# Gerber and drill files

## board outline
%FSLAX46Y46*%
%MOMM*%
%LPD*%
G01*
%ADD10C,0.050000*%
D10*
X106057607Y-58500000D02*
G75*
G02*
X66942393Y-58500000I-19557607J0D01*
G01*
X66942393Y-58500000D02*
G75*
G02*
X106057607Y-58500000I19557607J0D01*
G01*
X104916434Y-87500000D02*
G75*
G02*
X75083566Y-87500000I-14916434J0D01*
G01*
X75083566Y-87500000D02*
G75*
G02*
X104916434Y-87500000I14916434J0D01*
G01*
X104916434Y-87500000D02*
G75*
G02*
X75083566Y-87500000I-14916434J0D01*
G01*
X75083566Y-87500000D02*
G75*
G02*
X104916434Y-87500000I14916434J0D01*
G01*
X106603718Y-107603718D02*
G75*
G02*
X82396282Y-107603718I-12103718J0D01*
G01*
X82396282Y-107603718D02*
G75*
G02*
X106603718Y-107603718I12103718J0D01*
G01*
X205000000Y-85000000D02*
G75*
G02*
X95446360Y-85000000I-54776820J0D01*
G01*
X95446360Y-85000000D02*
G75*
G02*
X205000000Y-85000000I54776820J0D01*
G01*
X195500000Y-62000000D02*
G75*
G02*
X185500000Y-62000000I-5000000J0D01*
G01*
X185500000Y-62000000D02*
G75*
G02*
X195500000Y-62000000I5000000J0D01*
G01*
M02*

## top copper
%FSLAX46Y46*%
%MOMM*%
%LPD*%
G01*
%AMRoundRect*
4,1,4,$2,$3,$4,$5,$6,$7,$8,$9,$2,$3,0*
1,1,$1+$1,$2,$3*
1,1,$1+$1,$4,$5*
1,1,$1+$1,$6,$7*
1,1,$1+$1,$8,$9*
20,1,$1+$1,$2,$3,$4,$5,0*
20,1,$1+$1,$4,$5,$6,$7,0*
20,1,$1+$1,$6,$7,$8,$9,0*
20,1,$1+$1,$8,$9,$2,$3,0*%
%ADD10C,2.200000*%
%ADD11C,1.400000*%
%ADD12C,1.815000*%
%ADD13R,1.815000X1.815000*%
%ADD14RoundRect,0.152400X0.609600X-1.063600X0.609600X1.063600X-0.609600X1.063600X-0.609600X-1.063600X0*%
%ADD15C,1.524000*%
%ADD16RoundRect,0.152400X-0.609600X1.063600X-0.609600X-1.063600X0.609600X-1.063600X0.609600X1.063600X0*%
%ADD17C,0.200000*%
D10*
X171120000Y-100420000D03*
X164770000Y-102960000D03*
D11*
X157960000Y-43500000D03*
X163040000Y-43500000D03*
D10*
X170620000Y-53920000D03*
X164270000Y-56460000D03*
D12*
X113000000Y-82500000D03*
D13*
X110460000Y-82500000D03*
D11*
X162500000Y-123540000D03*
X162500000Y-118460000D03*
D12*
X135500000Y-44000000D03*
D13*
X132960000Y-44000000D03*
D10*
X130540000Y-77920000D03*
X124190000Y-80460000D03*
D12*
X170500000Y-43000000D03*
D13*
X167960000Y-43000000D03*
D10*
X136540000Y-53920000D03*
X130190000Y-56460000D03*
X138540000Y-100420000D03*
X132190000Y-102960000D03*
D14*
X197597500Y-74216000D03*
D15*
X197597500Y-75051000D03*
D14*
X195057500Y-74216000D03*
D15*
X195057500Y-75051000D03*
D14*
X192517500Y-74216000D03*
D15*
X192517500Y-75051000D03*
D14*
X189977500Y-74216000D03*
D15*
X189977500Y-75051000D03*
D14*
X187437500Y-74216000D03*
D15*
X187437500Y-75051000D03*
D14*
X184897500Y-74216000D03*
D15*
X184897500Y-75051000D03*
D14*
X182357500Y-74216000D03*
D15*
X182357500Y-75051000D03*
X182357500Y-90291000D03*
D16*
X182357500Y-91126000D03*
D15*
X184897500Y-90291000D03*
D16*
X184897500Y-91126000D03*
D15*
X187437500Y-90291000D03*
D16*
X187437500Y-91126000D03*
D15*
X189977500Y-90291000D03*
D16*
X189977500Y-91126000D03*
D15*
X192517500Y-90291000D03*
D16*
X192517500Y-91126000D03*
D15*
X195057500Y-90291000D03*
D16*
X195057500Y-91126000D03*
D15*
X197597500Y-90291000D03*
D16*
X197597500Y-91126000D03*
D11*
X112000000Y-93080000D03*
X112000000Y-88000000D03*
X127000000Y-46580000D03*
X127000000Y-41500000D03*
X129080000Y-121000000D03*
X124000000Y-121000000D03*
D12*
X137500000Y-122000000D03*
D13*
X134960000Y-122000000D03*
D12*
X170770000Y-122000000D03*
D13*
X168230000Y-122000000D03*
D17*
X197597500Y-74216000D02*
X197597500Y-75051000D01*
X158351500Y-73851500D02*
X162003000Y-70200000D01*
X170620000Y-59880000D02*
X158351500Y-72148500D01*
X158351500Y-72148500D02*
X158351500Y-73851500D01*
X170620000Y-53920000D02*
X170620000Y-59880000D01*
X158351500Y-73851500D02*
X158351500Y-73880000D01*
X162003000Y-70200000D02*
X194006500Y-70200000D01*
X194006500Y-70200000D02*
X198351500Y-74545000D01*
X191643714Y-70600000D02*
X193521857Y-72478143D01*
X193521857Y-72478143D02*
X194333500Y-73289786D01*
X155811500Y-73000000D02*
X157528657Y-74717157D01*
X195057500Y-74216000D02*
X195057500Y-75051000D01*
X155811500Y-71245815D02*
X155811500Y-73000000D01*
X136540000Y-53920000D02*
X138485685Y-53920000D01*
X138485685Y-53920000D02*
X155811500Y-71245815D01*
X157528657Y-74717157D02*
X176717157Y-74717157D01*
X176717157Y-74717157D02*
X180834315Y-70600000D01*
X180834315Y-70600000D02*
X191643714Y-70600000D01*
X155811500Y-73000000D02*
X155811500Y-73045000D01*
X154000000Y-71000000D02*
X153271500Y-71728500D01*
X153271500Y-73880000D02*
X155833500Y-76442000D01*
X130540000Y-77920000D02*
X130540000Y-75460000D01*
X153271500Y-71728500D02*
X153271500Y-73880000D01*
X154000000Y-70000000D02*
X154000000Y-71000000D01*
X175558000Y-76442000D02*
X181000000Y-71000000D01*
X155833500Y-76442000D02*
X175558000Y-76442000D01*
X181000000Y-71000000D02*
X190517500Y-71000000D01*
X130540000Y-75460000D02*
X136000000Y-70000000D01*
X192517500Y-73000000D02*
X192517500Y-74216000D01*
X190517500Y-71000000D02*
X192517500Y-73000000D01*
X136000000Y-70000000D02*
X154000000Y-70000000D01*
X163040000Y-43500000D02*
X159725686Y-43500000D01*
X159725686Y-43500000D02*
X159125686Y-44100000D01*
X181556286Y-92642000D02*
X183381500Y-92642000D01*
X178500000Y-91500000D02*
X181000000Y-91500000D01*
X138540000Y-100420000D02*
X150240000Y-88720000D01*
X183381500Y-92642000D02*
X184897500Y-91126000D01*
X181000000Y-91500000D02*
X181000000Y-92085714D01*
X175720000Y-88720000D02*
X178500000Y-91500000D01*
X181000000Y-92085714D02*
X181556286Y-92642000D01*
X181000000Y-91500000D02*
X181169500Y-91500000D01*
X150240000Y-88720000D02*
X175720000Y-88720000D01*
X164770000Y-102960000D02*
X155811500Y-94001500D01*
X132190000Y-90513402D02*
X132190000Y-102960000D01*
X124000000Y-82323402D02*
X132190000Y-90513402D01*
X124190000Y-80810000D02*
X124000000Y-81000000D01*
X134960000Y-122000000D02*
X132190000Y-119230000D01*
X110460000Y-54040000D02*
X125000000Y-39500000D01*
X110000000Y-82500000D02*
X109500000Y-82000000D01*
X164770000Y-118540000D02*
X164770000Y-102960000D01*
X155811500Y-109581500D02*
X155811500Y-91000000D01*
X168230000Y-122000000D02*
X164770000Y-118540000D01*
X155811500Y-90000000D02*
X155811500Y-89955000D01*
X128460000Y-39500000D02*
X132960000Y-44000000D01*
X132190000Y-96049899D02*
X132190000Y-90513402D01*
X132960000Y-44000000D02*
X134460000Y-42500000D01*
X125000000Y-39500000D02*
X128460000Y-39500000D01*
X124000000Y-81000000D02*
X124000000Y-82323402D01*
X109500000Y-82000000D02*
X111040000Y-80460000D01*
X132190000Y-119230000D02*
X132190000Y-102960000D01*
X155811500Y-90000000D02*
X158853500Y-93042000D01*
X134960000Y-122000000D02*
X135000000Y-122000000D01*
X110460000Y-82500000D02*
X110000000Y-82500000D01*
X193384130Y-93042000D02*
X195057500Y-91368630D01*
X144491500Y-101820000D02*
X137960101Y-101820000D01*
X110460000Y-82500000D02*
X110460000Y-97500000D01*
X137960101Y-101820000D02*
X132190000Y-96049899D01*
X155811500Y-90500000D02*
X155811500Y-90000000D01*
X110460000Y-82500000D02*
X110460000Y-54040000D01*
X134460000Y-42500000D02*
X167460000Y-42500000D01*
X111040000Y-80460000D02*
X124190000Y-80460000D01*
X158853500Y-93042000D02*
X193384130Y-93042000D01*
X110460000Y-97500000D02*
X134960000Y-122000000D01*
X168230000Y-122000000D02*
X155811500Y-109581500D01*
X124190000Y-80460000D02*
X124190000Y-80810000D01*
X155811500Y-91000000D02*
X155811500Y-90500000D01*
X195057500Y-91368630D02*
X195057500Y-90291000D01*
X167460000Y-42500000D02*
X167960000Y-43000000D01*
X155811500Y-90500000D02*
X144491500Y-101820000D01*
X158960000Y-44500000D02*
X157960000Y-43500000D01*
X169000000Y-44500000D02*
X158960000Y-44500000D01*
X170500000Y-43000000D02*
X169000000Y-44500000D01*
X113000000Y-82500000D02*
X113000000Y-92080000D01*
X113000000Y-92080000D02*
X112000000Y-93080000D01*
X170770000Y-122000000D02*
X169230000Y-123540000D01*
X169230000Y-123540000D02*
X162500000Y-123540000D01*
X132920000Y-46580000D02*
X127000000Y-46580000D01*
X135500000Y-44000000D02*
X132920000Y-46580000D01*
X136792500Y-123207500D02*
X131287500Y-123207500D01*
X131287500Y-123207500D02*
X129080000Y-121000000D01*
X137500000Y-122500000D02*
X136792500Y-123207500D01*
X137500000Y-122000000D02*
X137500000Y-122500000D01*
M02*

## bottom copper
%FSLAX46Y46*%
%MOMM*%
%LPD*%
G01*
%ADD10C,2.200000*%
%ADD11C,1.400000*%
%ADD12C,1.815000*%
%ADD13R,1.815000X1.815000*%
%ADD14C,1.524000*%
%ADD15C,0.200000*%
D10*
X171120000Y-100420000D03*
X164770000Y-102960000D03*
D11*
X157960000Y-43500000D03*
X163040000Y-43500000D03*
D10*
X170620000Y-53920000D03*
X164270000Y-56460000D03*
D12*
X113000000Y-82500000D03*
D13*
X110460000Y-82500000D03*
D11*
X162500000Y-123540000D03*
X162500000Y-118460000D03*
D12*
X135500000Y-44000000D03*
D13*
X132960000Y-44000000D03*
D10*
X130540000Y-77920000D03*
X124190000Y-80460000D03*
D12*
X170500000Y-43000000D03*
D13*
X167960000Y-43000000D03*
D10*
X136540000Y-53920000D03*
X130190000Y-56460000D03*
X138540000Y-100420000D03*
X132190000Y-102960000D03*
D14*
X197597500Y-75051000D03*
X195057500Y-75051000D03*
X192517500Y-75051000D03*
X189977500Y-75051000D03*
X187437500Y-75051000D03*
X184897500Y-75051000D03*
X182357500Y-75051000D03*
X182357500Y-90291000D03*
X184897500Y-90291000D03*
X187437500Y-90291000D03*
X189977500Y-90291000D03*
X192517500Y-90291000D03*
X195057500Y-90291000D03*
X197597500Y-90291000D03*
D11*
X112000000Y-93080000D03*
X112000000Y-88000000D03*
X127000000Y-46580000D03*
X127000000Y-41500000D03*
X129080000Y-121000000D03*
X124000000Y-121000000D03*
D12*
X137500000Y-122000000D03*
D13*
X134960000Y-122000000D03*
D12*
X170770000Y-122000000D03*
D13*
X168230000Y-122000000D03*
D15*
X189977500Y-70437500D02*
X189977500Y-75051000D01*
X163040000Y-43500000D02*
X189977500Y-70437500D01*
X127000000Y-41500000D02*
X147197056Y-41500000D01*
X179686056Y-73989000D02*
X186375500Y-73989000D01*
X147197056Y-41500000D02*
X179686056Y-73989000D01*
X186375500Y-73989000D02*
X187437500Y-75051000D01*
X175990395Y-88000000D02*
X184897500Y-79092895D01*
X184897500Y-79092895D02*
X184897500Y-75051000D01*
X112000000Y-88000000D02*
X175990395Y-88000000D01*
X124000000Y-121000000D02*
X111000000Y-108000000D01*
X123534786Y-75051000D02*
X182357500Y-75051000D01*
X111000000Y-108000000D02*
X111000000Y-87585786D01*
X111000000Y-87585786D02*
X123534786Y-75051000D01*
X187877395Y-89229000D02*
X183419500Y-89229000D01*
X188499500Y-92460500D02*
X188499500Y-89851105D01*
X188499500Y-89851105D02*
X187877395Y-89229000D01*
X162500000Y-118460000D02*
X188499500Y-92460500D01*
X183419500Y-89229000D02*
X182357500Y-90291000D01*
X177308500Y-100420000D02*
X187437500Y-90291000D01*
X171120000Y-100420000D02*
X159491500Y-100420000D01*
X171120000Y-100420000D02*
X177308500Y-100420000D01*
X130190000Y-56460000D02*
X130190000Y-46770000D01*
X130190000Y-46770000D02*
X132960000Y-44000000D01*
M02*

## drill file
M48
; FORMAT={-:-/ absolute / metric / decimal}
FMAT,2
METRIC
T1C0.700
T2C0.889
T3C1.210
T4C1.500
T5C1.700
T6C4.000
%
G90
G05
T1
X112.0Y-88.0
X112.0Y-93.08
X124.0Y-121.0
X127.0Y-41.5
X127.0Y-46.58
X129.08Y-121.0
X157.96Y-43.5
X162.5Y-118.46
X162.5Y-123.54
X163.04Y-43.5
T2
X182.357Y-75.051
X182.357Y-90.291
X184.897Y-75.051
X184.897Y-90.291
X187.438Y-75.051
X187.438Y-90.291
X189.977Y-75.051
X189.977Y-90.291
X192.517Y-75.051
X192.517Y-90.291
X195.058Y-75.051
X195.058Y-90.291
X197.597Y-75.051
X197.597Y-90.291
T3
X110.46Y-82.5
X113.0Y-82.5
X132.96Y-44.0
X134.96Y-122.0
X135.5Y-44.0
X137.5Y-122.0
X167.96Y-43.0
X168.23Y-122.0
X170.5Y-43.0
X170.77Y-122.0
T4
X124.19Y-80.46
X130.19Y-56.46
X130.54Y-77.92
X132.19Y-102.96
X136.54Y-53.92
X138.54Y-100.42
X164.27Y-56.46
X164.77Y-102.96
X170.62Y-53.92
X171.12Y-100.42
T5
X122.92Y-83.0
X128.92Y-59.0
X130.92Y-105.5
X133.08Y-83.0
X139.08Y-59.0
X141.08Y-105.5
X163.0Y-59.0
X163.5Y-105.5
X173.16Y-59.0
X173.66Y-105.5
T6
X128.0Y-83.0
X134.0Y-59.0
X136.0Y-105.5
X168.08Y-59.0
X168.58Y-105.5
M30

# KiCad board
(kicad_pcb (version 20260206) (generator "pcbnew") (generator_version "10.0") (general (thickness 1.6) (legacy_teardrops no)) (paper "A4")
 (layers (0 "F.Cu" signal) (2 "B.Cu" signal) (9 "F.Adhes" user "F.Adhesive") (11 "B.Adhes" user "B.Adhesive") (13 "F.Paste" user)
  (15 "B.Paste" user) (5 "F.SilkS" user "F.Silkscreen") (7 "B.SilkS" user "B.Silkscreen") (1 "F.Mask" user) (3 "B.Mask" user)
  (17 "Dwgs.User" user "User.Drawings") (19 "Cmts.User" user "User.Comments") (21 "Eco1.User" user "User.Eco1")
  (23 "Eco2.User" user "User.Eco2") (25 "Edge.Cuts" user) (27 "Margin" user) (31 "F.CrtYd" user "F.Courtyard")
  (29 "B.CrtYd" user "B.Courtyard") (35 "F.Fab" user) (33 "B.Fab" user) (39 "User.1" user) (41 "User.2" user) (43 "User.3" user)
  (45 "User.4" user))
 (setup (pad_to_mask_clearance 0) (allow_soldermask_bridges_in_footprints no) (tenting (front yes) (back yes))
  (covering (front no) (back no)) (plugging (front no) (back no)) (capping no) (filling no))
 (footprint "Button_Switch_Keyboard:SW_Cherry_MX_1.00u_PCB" (layer "F.Cu") (at 171.12 100.42)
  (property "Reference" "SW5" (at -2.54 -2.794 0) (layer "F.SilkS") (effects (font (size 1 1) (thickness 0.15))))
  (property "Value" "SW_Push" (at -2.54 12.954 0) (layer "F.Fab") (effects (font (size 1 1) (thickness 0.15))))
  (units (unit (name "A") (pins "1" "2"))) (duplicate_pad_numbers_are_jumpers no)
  (pad "" np_thru_hole circle (at -7.62 5.08) (size 1.7 1.7) (drill 1.7) (layers "*.Cu" "*.Mask"))
  (pad "" np_thru_hole circle (at -2.54 5.08) (size 4 4) (drill 4) (layers "*.Cu" "*.Mask"))
  (pad "" np_thru_hole circle (at 2.54 5.08) (size 1.7 1.7) (drill 1.7) (layers "*.Cu" "*.Mask"))
  (pad "1" thru_hole circle (at 0 0) (size 2.2 2.2) (drill 1.5) (layers "*.Cu" "*.Mask") (remove_unused_layers no) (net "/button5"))
  (pad "2" thru_hole circle (at -6.35 2.54) (size 2.2 2.2) (drill 1.5) (layers "*.Cu" "*.Mask") (remove_unused_layers no) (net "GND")))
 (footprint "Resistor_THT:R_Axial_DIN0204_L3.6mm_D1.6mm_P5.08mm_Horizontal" (layer "F.Cu") (at 157.96 43.5)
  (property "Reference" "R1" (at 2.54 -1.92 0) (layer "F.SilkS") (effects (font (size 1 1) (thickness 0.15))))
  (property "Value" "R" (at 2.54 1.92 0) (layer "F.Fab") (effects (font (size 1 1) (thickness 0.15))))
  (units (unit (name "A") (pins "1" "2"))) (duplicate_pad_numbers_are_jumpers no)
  (pad "1" thru_hole circle (at 0 0) (size 1.4 1.4) (drill 0.7) (layers "*.Cu" "*.Mask") (remove_unused_layers no) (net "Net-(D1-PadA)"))
  (pad "2" thru_hole circle (at 5.08 0) (size 1.4 1.4) (drill 0.7) (layers "*.Cu" "*.Mask") (remove_unused_layers no) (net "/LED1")))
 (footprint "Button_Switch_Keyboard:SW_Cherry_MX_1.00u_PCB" (layer "F.Cu") (at 170.62 53.92)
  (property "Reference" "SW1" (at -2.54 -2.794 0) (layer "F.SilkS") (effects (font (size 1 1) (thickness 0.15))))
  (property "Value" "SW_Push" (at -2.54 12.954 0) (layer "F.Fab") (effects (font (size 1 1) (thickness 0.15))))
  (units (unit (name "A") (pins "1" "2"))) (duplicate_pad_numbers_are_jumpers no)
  (pad "" np_thru_hole circle (at -7.62 5.08) (size 1.7 1.7) (drill 1.7) (layers "*.Cu" "*.Mask"))
  (pad "" np_thru_hole circle (at -2.54 5.08) (size 4 4) (drill 4) (layers "*.Cu" "*.Mask"))
  (pad "" np_thru_hole circle (at 2.54 5.08) (size 1.7 1.7) (drill 1.7) (layers "*.Cu" "*.Mask"))
  (pad "1" thru_hole circle (at 0 0) (size 2.2 2.2) (drill 1.5) (layers "*.Cu" "*.Mask") (remove_unused_layers no) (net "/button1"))
  (pad "2" thru_hole circle (at -6.35 2.54) (size 2.2 2.2) (drill 1.5) (layers "*.Cu" "*.Mask") (remove_unused_layers no) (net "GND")))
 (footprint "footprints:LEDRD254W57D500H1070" (layer "F.Cu") (at 111.73 82.5)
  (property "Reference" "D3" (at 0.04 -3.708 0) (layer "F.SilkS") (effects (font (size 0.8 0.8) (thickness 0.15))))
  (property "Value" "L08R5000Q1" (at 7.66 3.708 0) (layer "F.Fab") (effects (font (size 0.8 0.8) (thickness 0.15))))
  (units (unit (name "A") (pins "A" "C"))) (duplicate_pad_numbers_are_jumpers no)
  (pad "A" thru_hole circle (at 1.27 0) (size 1.815 1.815) (drill 1.21) (layers "*.Cu" "*.Mask") (remove_unused_layers no)
   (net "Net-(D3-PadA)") (solder_mask_margin 0.102))
  (pad "C" thru_hole rect (at -1.27 0) (size 1.815 1.815) (drill 1.21) (layers "*.Cu" "*.Mask") (remove_unused_layers no) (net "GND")
   (solder_mask_margin 0.102)))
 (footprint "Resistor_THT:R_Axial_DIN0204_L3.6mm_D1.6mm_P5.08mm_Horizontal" (layer "F.Cu") (at 162.5 123.54 90)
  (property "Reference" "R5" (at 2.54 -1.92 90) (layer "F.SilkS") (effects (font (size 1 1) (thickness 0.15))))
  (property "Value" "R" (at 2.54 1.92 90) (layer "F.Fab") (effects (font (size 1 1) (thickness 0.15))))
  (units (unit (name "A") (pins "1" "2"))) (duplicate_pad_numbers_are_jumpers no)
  (pad "1" thru_hole circle (at 0 0 90) (size 1.4 1.4) (drill 0.7) (layers "*.Cu" "*.Mask") (remove_unused_layers no) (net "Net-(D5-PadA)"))
  (pad "2" thru_hole circle (at 5.08 0 90) (size 1.4 1.4) (drill 0.7) (layers "*.Cu" "*.Mask") (remove_unused_layers no) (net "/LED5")))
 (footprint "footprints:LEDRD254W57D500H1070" (layer "F.Cu") (at 134.23 44)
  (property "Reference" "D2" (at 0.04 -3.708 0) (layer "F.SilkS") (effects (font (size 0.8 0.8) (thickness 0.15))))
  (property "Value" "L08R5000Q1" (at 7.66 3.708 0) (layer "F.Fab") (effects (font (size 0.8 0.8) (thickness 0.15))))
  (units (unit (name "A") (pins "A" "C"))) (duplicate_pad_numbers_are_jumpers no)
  (pad "A" thru_hole circle (at 1.27 0) (size 1.815 1.815) (drill 1.21) (layers "*.Cu" "*.Mask") (remove_unused_layers no)
   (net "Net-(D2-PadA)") (solder_mask_margin 0.102))
  (pad "C" thru_hole rect (at -1.27 0) (size 1.815 1.815) (drill 1.21) (layers "*.Cu" "*.Mask") (remove_unused_layers no) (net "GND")
   (solder_mask_margin 0.102)))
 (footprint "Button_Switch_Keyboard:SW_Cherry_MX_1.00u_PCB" (layer "F.Cu") (at 130.54 77.92)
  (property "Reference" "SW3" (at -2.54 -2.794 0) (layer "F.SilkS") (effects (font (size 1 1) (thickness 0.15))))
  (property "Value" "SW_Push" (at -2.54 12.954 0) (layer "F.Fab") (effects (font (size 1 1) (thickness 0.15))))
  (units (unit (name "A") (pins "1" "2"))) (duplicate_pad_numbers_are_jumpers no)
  (pad "" np_thru_hole circle (at -7.62 5.08) (size 1.7 1.7) (drill 1.7) (layers "*.Cu" "*.Mask"))
  (pad "" np_thru_hole circle (at -2.54 5.08) (size 4 4) (drill 4) (layers "*.Cu" "*.Mask"))
  (pad "" np_thru_hole circle (at 2.54 5.08) (size 1.7 1.7) (drill 1.7) (layers "*.Cu" "*.Mask"))
  (pad "1" thru_hole circle (at 0 0) (size 2.2 2.2) (drill 1.5) (layers "*.Cu" "*.Mask") (remove_unused_layers no) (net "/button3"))
  (pad "2" thru_hole circle (at -6.35 2.54) (size 2.2 2.2) (drill 1.5) (layers "*.Cu" "*.Mask") (remove_unused_layers no) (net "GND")))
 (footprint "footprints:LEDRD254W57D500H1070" (layer "F.Cu") (at 169.23 43)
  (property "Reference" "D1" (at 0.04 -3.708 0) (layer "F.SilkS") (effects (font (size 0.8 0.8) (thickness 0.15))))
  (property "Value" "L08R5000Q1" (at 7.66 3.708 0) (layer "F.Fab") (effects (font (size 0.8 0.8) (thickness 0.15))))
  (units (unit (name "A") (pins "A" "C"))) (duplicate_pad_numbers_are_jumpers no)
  (pad "A" thru_hole circle (at 1.27 0) (size 1.815 1.815) (drill 1.21) (layers "*.Cu" "*.Mask") (remove_unused_layers no)
   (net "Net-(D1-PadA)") (solder_mask_margin 0.102))
  (pad "C" thru_hole rect (at -1.27 0) (size 1.815 1.815) (drill 1.21) (layers "*.Cu" "*.Mask") (remove_unused_layers no) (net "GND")
   (solder_mask_margin 0.102)))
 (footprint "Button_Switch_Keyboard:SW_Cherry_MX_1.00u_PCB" (layer "F.Cu") (at 136.54 53.92)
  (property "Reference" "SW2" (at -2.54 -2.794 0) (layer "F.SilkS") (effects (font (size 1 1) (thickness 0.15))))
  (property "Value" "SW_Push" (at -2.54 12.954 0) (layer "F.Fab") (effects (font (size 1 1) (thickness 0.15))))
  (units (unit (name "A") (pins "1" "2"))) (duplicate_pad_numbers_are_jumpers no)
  (pad "" np_thru_hole circle (at -7.62 5.08) (size 1.7 1.7) (drill 1.7) (layers "*.Cu" "*.Mask"))
  (pad "" np_thru_hole circle (at -2.54 5.08) (size 4 4) (drill 4) (layers "*.Cu" "*.Mask"))
  (pad "" np_thru_hole circle (at 2.54 5.08) (size 1.7 1.7) (drill 1.7) (layers "*.Cu" "*.Mask"))
  (pad "1" thru_hole circle (at 0 0) (size 2.2 2.2) (drill 1.5) (layers "*.Cu" "*.Mask") (remove_unused_layers no) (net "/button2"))
  (pad "2" thru_hole circle (at -6.35 2.54) (size 2.2 2.2) (drill 1.5) (layers "*.Cu" "*.Mask") (remove_unused_layers no) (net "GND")))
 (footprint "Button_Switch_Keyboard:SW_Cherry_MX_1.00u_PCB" (layer "F.Cu") (at 138.54 100.42)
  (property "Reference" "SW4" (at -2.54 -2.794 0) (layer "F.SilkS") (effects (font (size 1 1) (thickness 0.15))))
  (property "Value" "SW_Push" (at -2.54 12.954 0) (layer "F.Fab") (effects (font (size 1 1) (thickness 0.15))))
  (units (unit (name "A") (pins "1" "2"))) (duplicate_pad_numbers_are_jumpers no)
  (pad "" np_thru_hole circle (at -7.62 5.08) (size 1.7 1.7) (drill 1.7) (layers "*.Cu" "*.Mask"))
  (pad "" np_thru_hole circle (at -2.54 5.08) (size 4 4) (drill 4) (layers "*.Cu" "*.Mask"))
  (pad "" np_thru_hole circle (at 2.54 5.08) (size 1.7 1.7) (drill 1.7) (layers "*.Cu" "*.Mask"))
  (pad "1" thru_hole circle (at 0 0) (size 2.2 2.2) (drill 1.5) (layers "*.Cu" "*.Mask") (remove_unused_layers no) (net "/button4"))
  (pad "2" thru_hole circle (at -6.35 2.54) (size 2.2 2.2) (drill 1.5) (layers "*.Cu" "*.Mask") (remove_unused_layers no) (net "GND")))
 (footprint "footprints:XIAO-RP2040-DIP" (layer "F.Cu") (at 189.9775 82.671)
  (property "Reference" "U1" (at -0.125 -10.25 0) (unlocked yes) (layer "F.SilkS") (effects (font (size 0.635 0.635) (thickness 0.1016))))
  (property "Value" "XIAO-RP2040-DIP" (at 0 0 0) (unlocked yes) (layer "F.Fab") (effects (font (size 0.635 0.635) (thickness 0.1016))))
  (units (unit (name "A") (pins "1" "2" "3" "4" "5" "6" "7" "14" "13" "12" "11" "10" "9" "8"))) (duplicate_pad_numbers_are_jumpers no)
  (pad "1" smd roundrect (at 7.62 -8.455 90) (size 2.432 1.524) (layers "F.Cu" "F.Mask") (roundrect_rratio 0.1) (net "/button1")
   (thermal_bridge_angle 45))
  (pad "1" thru_hole circle (at 7.62 -7.62 90) (size 1.524 1.524) (drill 0.889) (layers "*.Cu" "*.Mask") (remove_unused_layers no)
   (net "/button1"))
  (pad "2" smd roundrect (at 5.08 -8.455 90) (size 2.432 1.524) (layers "F.Cu" "F.Mask") (roundrect_rratio 0.1) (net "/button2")
   (thermal_bridge_angle 45))
  (pad "2" thru_hole circle (at 5.08 -7.62 90) (size 1.524 1.524) (drill 0.889) (layers "*.Cu" "*.Mask") (remove_unused_layers no)
   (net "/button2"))
  (pad "3" smd roundrect (at 2.54 -8.455 90) (size 2.432 1.524) (layers "F.Cu" "F.Mask") (roundrect_rratio 0.1) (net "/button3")
   (thermal_bridge_angle 45))
  (pad "3" thru_hole circle (at 2.54 -7.62 90) (size 1.524 1.524) (drill 0.889) (layers "*.Cu" "*.Mask") (remove_unused_layers no)
   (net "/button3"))
  (pad "4" smd roundrect (at 0 -8.455 90) (size 2.432 1.524) (layers "F.Cu" "F.Mask") (roundrect_rratio 0.1) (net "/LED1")
   (thermal_bridge_angle 45))
  (pad "4" thru_hole circle (at 0 -7.62 90) (size 1.524 1.524) (drill 0.889) (layers "*.Cu" "*.Mask") (remove_unused_layers no)
   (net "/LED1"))
  (pad "5" smd roundrect (at -2.54 -8.455 90) (size 2.432 1.524) (layers "F.Cu" "F.Mask") (roundrect_rratio 0.1) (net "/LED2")
   (thermal_bridge_angle 45))
  (pad "5" thru_hole circle (at -2.54 -7.62 90) (size 1.524 1.524) (drill 0.889) (layers "*.Cu" "*.Mask") (remove_unused_layers no)
   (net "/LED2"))
  (pad "6" smd roundrect (at -5.08 -8.455 90) (size 2.432 1.524) (layers "F.Cu" "F.Mask") (roundrect_rratio 0.1) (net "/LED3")
   (thermal_bridge_angle 45))
  (pad "6" thru_hole circle (at -5.08 -7.62 90) (size 1.524 1.524) (drill 0.889) (layers "*.Cu" "*.Mask") (remove_unused_layers no)
   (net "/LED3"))
  (pad "7" smd roundrect (at -7.62 -8.455 90) (size 2.432 1.524) (layers "F.Cu" "F.Mask") (roundrect_rratio 0.1) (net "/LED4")
   (thermal_bridge_angle 45))
  (pad "7" thru_hole circle (at -7.62 -7.62 90) (size 1.524 1.524) (drill 0.889) (layers "*.Cu" "*.Mask") (remove_unused_layers no)
   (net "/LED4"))
  (pad "8" thru_hole circle (at -7.62 7.62 270) (size 1.524 1.524) (drill 0.889) (layers "*.Cu" "*.Mask") (remove_unused_layers no)
   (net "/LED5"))
  (pad "8" smd roundrect (at -7.62 8.455 270) (size 2.432 1.524) (layers "F.Cu" "F.Mask") (roundrect_rratio 0.1) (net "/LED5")
   (thermal_bridge_angle 45))
  (pad "9" thru_hole circle (at -5.08 7.62 270) (size 1.524 1.524) (drill 0.889) (layers "*.Cu" "*.Mask") (remove_unused_layers no)
   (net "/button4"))
  (pad "9" smd roundrect (at -5.08 8.455 270) (size 2.432 1.524) (layers "F.Cu" "F.Mask") (roundrect_rratio 0.1) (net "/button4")
   (thermal_bridge_angle 45))
  (pad "10" thru_hole circle (at -2.54 7.62 270) (size 1.524 1.524) (drill 0.889) (layers "*.Cu" "*.Mask") (remove_unused_layers no)
   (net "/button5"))
  (pad "10" smd roundrect (at -2.54 8.455 270) (size 2.432 1.524) (layers "F.Cu" "F.Mask") (roundrect_rratio 0.1) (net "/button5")
   (thermal_bridge_angle 45))
  (pad "11" thru_hole circle (at 0 7.62 270) (size 1.524 1.524) (drill 0.889) (layers "*.Cu" "*.Mask") (remove_unused_layers no)
   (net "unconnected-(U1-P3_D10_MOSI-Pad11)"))
  (pad "11" smd roundrect (at 0 8.455 270) (size 2.432 1.524) (layers "F.Cu" "F.Mask") (roundrect_rratio 0.1)
   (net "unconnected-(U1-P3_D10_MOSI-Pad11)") (thermal_bridge_angle 45))
  (pad "12" thru_hole circle (at 2.54 7.62 270) (size 1.524 1.524) (drill 0.889) (layers "*.Cu" "*.Mask") (remove_unused_layers no)
   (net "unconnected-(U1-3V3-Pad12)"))
  (pad "12" smd roundrect (at 2.54 8.455 270) (size 2.432 1.524) (layers "F.Cu" "F.Mask") (roundrect_rratio 0.1)
   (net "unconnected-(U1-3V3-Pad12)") (thermal_bridge_angle 45))
  (pad "13" thru_hole circle (at 5.08 7.62 270) (size 1.524 1.524) (drill 0.889) (layers "*.Cu" "*.Mask") (remove_unused_layers no)
   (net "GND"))
  (pad "13" smd roundrect (at 5.08 8.455 270) (size 2.432 1.524) (layers "F.Cu" "F.Mask") (roundrect_rratio 0.1) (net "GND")
   (thermal_bridge_angle 45))
  (pad "14" thru_hole circle (at 7.62 7.62 270) (size 1.524 1.524) (drill 0.889) (layers "*.Cu" "*.Mask") (remove_unused_layers no)
   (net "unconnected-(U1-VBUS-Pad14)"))
  (pad "14" smd roundrect (at 7.62 8.455 270) (size 2.432 1.524) (layers "F.Cu" "F.Mask") (roundrect_rratio 0.1)
   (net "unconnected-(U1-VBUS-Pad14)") (thermal_bridge_angle 45)))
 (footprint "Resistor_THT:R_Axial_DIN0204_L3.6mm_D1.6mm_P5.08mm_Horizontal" (layer "F.Cu") (at 112 93.08 90)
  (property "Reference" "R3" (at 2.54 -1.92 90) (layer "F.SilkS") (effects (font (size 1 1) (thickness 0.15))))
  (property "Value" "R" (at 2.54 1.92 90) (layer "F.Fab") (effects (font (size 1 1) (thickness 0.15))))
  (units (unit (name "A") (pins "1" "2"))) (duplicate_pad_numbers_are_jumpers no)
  (pad "1" thru_hole circle (at 0 0 90) (size 1.4 1.4) (drill 0.7) (layers "*.Cu" "*.Mask") (remove_unused_layers no) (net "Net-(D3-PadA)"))
  (pad "2" thru_hole circle (at 5.08 0 90) (size 1.4 1.4) (drill 0.7) (layers "*.Cu" "*.Mask") (remove_unused_layers no) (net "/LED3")))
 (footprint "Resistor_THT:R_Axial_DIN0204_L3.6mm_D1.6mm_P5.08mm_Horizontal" (layer "F.Cu") (at 127 46.58 90)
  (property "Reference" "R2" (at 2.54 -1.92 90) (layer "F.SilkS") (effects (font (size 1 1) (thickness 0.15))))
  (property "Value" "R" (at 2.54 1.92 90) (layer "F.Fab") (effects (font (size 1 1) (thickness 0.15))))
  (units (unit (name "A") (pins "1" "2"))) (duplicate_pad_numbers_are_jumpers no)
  (pad "1" thru_hole circle (at 0 0 90) (size 1.4 1.4) (drill 0.7) (layers "*.Cu" "*.Mask") (remove_unused_layers no) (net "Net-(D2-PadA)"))
  (pad "2" thru_hole circle (at 5.08 0 90) (size 1.4 1.4) (drill 0.7) (layers "*.Cu" "*.Mask") (remove_unused_layers no) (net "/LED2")))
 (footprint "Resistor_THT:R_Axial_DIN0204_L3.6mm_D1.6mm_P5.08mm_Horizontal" (layer "F.Cu") (at 129.08 121 180)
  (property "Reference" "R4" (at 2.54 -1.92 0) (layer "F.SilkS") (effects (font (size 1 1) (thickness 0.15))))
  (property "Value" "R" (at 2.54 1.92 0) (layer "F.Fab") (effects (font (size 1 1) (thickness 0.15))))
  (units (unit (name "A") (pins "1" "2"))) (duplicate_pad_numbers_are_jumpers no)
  (pad "1" thru_hole circle (at 0 0 180) (size 1.4 1.4) (drill 0.7) (layers "*.Cu" "*.Mask") (remove_unused_layers no) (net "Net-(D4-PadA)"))
  (pad "2" thru_hole circle (at 5.08 0 180) (size 1.4 1.4) (drill 0.7) (layers "*.Cu" "*.Mask") (remove_unused_layers no) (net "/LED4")))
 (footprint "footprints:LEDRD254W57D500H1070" (layer "F.Cu") (at 136.23 122)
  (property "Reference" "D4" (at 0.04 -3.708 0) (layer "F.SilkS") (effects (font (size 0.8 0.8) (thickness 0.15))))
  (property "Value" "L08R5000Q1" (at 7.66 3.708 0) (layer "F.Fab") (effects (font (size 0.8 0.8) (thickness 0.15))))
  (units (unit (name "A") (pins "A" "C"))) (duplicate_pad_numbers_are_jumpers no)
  (pad "A" thru_hole circle (at 1.27 0) (size 1.815 1.815) (drill 1.21) (layers "*.Cu" "*.Mask") (remove_unused_layers no)
   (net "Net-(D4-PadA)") (solder_mask_margin 0.102))
  (pad "C" thru_hole rect (at -1.27 0) (size 1.815 1.815) (drill 1.21) (layers "*.Cu" "*.Mask") (remove_unused_layers no) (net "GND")
   (solder_mask_margin 0.102)))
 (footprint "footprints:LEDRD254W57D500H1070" (layer "F.Cu") (at 169.5 122)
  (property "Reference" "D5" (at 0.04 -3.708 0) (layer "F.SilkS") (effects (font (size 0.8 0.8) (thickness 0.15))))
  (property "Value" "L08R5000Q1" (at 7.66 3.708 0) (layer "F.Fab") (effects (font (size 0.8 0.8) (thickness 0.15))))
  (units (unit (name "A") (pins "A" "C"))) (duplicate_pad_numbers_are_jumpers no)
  (pad "A" thru_hole circle (at 1.27 0) (size 1.815 1.815) (drill 1.21) (layers "*.Cu" "*.Mask") (remove_unused_layers no)
   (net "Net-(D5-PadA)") (solder_mask_margin 0.102))
  (pad "C" thru_hole rect (at -1.27 0) (size 1.815 1.815) (drill 1.21) (layers "*.Cu" "*.Mask") (remove_unused_layers no) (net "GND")
   (solder_mask_margin 0.102)))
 (gr_circle (center 86.5 58.5) (end 103 48) (stroke (width 0.05) (type default)) (fill no) (layer "Edge.Cuts"))
 (gr_circle (center 90 87.5) (end 90 72.583566) (stroke (width 0.05) (type default)) (fill no) (layer "Edge.Cuts"))
 (gr_circle (center 90 87.5) (end 93.5 73) (stroke (width 0.05) (type default)) (fill no) (layer "Edge.Cuts"))
 (gr_circle (center 94.5 107.603718) (end 102 98.103718) (stroke (width 0.05) (type default)) (fill no) (layer "Edge.Cuts"))
 (gr_circle (center 150.22318 85) (end 180.72318 39.5) (stroke (width 0.05) (type default)) (fill no) (layer "Edge.Cuts"))
 (gr_circle (center 190.5 62) (end 194.5 59) (stroke (width 0.05) (type default)) (fill no) (layer "Edge.Cuts"))
 (segment (start 197.5975 74.216) (end 197.5975 75.051) (width 0.2) (layer "F.Cu") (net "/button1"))
 (segment (start 158.3515 73.8515) (end 162.003 70.2) (width 0.2) (layer "F.Cu") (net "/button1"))
 (segment (start 170.62 59.88) (end 158.3515 72.1485) (width 0.2) (layer "F.Cu") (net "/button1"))
 (segment (start 158.3515 72.1485) (end 158.3515 73.8515) (width 0.2) (layer "F.Cu") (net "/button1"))
 (segment (start 170.62 53.92) (end 170.62 59.88) (width 0.2) (layer "F.Cu") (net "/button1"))
 (segment (start 158.3515 73.8515) (end 158.3515 73.88) (width 0.2) (layer "F.Cu") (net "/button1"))
 (segment (start 162.003 70.2) (end 194.0065 70.2) (width 0.2) (layer "F.Cu") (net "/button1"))
 (segment (start 194.0065 70.2) (end 198.3515 74.545) (width 0.2) (layer "F.Cu") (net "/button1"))
 (segment (start 191.643714 70.6) (end 193.521857 72.478143) (width 0.2) (layer "F.Cu") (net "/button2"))
 (segment (start 193.521857 72.478143) (end 194.3335 73.289786) (width 0.2) (layer "F.Cu") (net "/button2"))
 (segment (start 155.8115 73) (end 157.528657 74.717157) (width 0.2) (layer "F.Cu") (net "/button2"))
 (segment (start 195.0575 74.216) (end 195.0575 75.051) (width 0.2) (layer "F.Cu") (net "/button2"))
 (segment (start 155.8115 71.245815) (end 155.8115 73) (width 0.2) (layer "F.Cu") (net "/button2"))
 (segment (start 136.54 53.92) (end 138.485685 53.92) (width 0.2) (layer "F.Cu") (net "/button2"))
 (segment (start 138.485685 53.92) (end 155.8115 71.245815) (width 0.2) (layer "F.Cu") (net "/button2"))
 (segment (start 157.528657 74.717157) (end 176.717157 74.717157) (width 0.2) (layer "F.Cu") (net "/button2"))
 (segment (start 176.717157 74.717157) (end 180.834315 70.6) (width 0.2) (layer "F.Cu") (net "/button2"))
 (segment (start 180.834315 70.6) (end 191.643714 70.6) (width 0.2) (layer "F.Cu") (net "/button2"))
 (segment (start 155.8115 73) (end 155.8115 73.045) (width 0.2) (layer "F.Cu") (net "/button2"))
 (segment (start 154 71) (end 153.2715 71.7285) (width 0.2) (layer "F.Cu") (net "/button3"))
 (segment (start 153.2715 73.88) (end 155.8335 76.442) (width 0.2) (layer "F.Cu") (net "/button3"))
 (segment (start 130.54 77.92) (end 130.54 75.46) (width 0.2) (layer "F.Cu") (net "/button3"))
 (segment (start 153.2715 71.7285) (end 153.2715 73.88) (width 0.2) (layer "F.Cu") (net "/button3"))
 (segment (start 154 70) (end 154 71) (width 0.2) (layer "F.Cu") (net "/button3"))
 (segment (start 175.558 76.442) (end 181 71) (width 0.2) (layer "F.Cu") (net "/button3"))
 (segment (start 155.8335 76.442) (end 175.558 76.442) (width 0.2) (layer "F.Cu") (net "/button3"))
 (segment (start 181 71) (end 190.5175 71) (width 0.2) (layer "F.Cu") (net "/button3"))
 (segment (start 130.54 75.46) (end 136 70) (width 0.2) (layer "F.Cu") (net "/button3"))
 (segment (start 192.5175 73) (end 192.5175 74.216) (width 0.2) (layer "F.Cu") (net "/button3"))
 (segment (start 190.5175 71) (end 192.5175 73) (width 0.2) (layer "F.Cu") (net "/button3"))
 (segment (start 136 70) (end 154 70) (width 0.2) (layer "F.Cu") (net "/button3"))
 (segment (start 163.04 43.5) (end 159.725686 43.5) (width 0.2) (layer "F.Cu") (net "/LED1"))
 (segment (start 159.725686 43.5) (end 159.125686 44.1) (width 0.2) (layer "F.Cu") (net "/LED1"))
 (segment (start 189.9775 70.4375) (end 189.9775 75.051) (width 0.2) (layer "B.Cu") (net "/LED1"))
 (segment (start 163.04 43.5) (end 189.9775 70.4375) (width 0.2) (layer "B.Cu") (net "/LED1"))
 (segment (start 127 41.5) (end 147.197056 41.5) (width 0.2) (layer "B.Cu") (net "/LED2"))
 (segment (start 179.686056 73.989) (end 186.3755 73.989) (width 0.2) (layer "B.Cu") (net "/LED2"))
 (segment (start 147.197056 41.5) (end 179.686056 73.989) (width 0.2) (layer "B.Cu") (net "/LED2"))
 (segment (start 186.3755 73.989) (end 187.4375 75.051) (width 0.2) (layer "B.Cu") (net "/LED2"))
 (segment (start 175.990395 88) (end 184.8975 79.092895) (width 0.2) (layer "B.Cu") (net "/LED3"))
 (segment (start 184.8975 79.092895) (end 184.8975 75.051) (width 0.2) (layer "B.Cu") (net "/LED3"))
 (segment (start 112 88) (end 175.990395 88) (width 0.2) (layer "B.Cu") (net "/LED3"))
 (segment (start 124 121) (end 111 108) (width 0.2) (layer "B.Cu") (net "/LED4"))
 (segment (start 123.534786 75.051) (end 182.3575 75.051) (width 0.2) (layer "B.Cu") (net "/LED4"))
 (segment (start 111 108) (end 111 87.585786) (width 0.2) (layer "B.Cu") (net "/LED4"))
 (segment (start 111 87.585786) (end 123.534786 75.051) (width 0.2) (layer "B.Cu") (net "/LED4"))
 (segment (start 187.877395 89.229) (end 183.4195 89.229) (width 0.2) (layer "B.Cu") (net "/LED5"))
 (segment (start 188.4995 92.4605) (end 188.4995 89.851105) (width 0.2) (layer "B.Cu") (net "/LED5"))
 (segment (start 188.4995 89.851105) (end 187.877395 89.229) (width 0.2) (layer "B.Cu") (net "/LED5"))
 (segment (start 162.5 118.46) (end 188.4995 92.4605) (width 0.2) (layer "B.Cu") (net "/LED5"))
 (segment (start 183.4195 89.229) (end 182.3575 90.291) (width 0.2) (layer "B.Cu") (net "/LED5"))
 (segment (start 181.556286 92.642) (end 183.3815 92.642) (width 0.2) (layer "F.Cu") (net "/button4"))
 (segment (start 178.5 91.5) (end 181 91.5) (width 0.2) (layer "F.Cu") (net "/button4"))
 (segment (start 138.54 100.42) (end 150.24 88.72) (width 0.2) (layer "F.Cu") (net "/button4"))
 (segment (start 183.3815 92.642) (end 184.8975 91.126) (width 0.2) (layer "F.Cu") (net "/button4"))
 (segment (start 181 91.5) (end 181 92.085714) (width 0.2) (layer "F.Cu") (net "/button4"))
 (segment (start 175.72 88.72) (end 178.5 91.5) (width 0.2) (layer "F.Cu") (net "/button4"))
 (segment (start 181 92.085714) (end 181.556286 92.642) (width 0.2) (layer "F.Cu") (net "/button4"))
 (segment (start 181 91.5) (end 181.1695 91.5) (width 0.2) (layer "F.Cu") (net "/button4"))
 (segment (start 150.24 88.72) (end 175.72 88.72) (width 0.2) (layer "F.Cu") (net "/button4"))
 (segment (start 177.3085 100.42) (end 187.4375 90.291) (width 0.2) (layer "B.Cu") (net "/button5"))
 (segment (start 171.12 100.42) (end 159.4915 100.42) (width 0.2) (layer "B.Cu") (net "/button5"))
 (segment (start 171.12 100.42) (end 177.3085 100.42) (width 0.2) (layer "B.Cu") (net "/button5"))
 (segment (start 164.77 102.96) (end 155.8115 94.0015) (width 0.2) (layer "F.Cu") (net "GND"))
 (segment (start 132.19 90.513402) (end 132.19 102.96) (width 0.2) (layer "F.Cu") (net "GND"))
 (segment (start 124 82.323402) (end 132.19 90.513402) (width 0.2) (layer "F.Cu") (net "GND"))
 (segment (start 124.19 80.81) (end 124 81) (width 0.2) (layer "F.Cu") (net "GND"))
 (segment (start 134.96 122) (end 132.19 119.23) (width 0.2) (layer "F.Cu") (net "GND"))
 (segment (start 110.46 54.04) (end 125 39.5) (width 0.2) (layer "F.Cu") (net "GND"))
 (segment (start 110 82.5) (end 109.5 82) (width 0.2) (layer "F.Cu") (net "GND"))
 (segment (start 164.77 118.54) (end 164.77 102.96) (width 0.2) (layer "F.Cu") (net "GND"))
 (segment (start 155.8115 109.5815) (end 155.8115 91) (width 0.2) (layer "F.Cu") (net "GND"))
 (segment (start 168.23 122) (end 164.77 118.54) (width 0.2) (layer "F.Cu") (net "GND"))
 (segment (start 155.8115 90) (end 155.8115 89.955) (width 0.2) (layer "F.Cu") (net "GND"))
 (segment (start 128.46 39.5) (end 132.96 44) (width 0.2) (layer "F.Cu") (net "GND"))
 (segment (start 132.19 96.049899) (end 132.19 90.513402) (width 0.2) (layer "F.Cu") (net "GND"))
 (segment (start 132.96 44) (end 134.46 42.5) (width 0.2) (layer "F.Cu") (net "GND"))
 (segment (start 125 39.5) (end 128.46 39.5) (width 0.2) (layer "F.Cu") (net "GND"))
 (segment (start 124 81) (end 124 82.323402) (width 0.2) (layer "F.Cu") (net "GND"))
 (segment (start 109.5 82) (end 111.04 80.46) (width 0.2) (layer "F.Cu") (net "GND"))
 (segment (start 132.19 119.23) (end 132.19 102.96) (width 0.2) (layer "F.Cu") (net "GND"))
 (segment (start 155.8115 90) (end 158.8535 93.042) (width 0.2) (layer "F.Cu") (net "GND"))
 (segment (start 134.96 122) (end 135 122) (width 0.2) (layer "F.Cu") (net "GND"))
 (segment (start 110.46 82.5) (end 110 82.5) (width 0.2) (layer "F.Cu") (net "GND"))
 (segment (start 193.38413 93.042) (end 195.0575 91.36863) (width 0.2) (layer "F.Cu") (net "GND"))
 (segment (start 144.4915 101.82) (end 137.960101 101.82) (width 0.2) (layer "F.Cu") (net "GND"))
 (segment (start 110.46 82.5) (end 110.46 97.5) (width 0.2) (layer "F.Cu") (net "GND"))
 (segment (start 137.960101 101.82) (end 132.19 96.049899) (width 0.2) (layer "F.Cu") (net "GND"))
 (segment (start 155.8115 90.5) (end 155.8115 90) (width 0.2) (layer "F.Cu") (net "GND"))
 (segment (start 110.46 82.5) (end 110.46 54.04) (width 0.2) (layer "F.Cu") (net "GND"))
 (segment (start 134.46 42.5) (end 167.46 42.5) (width 0.2) (layer "F.Cu") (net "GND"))
 (segment (start 111.04 80.46) (end 124.19 80.46) (width 0.2) (layer "F.Cu") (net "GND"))
 (segment (start 158.8535 93.042) (end 193.38413 93.042) (width 0.2) (layer "F.Cu") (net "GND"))
 (segment (start 110.46 97.5) (end 134.96 122) (width 0.2) (layer "F.Cu") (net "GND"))
 (segment (start 168.23 122) (end 155.8115 109.5815) (width 0.2) (layer "F.Cu") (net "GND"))
 (segment (start 124.19 80.46) (end 124.19 80.81) (width 0.2) (layer "F.Cu") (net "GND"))
 (segment (start 155.8115 91) (end 155.8115 90.5) (width 0.2) (layer "F.Cu") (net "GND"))
 (segment (start 195.0575 91.36863) (end 195.0575 90.291) (width 0.2) (layer "F.Cu") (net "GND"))
 (segment (start 167.46 42.5) (end 167.96 43) (width 0.2) (layer "F.Cu") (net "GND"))
 (segment (start 155.8115 90.5) (end 144.4915 101.82) (width 0.2) (layer "F.Cu") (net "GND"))
 (segment (start 130.19 56.46) (end 130.19 46.77) (width 0.2) (layer "B.Cu") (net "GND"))
 (segment (start 130.19 46.77) (end 132.96 44) (width 0.2) (layer "B.Cu") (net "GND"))
 (segment (start 158.96 44.5) (end 157.96 43.5) (width 0.2) (layer "F.Cu") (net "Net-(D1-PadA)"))
 (segment (start 169 44.5) (end 158.96 44.5) (width 0.2) (layer "F.Cu") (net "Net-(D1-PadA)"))
 (segment (start 170.5 43) (end 169 44.5) (width 0.2) (layer "F.Cu") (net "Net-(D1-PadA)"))
 (segment (start 113 82.5) (end 113 92.08) (width 0.2) (layer "F.Cu") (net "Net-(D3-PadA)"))
 (segment (start 113 92.08) (end 112 93.08) (width 0.2) (layer "F.Cu") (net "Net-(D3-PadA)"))
 (segment (start 170.77 122) (end 169.23 123.54) (width 0.2) (layer "F.Cu") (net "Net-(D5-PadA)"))
 (segment (start 169.23 123.54) (end 162.5 123.54) (width 0.2) (layer "F.Cu") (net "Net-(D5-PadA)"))
 (segment (start 132.92 46.58) (end 127 46.58) (width 0.2) (layer "F.Cu") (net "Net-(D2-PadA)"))
 (segment (start 135.5 44) (end 132.92 46.58) (width 0.2) (layer "F.Cu") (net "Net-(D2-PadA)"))
 (segment (start 136.7925 123.2075) (end 131.2875 123.2075) (width 0.2) (layer "F.Cu") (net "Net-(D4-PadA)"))
 (segment (start 131.2875 123.2075) (end 129.08 121) (width 0.2) (layer "F.Cu") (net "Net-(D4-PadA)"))
 (segment (start 137.5 122.5) (end 136.7925 123.2075) (width 0.2) (layer "F.Cu") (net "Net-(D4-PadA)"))
 (segment (start 137.5 122) (end 137.5 122.5) (width 0.2) (layer "F.Cu") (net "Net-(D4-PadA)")))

